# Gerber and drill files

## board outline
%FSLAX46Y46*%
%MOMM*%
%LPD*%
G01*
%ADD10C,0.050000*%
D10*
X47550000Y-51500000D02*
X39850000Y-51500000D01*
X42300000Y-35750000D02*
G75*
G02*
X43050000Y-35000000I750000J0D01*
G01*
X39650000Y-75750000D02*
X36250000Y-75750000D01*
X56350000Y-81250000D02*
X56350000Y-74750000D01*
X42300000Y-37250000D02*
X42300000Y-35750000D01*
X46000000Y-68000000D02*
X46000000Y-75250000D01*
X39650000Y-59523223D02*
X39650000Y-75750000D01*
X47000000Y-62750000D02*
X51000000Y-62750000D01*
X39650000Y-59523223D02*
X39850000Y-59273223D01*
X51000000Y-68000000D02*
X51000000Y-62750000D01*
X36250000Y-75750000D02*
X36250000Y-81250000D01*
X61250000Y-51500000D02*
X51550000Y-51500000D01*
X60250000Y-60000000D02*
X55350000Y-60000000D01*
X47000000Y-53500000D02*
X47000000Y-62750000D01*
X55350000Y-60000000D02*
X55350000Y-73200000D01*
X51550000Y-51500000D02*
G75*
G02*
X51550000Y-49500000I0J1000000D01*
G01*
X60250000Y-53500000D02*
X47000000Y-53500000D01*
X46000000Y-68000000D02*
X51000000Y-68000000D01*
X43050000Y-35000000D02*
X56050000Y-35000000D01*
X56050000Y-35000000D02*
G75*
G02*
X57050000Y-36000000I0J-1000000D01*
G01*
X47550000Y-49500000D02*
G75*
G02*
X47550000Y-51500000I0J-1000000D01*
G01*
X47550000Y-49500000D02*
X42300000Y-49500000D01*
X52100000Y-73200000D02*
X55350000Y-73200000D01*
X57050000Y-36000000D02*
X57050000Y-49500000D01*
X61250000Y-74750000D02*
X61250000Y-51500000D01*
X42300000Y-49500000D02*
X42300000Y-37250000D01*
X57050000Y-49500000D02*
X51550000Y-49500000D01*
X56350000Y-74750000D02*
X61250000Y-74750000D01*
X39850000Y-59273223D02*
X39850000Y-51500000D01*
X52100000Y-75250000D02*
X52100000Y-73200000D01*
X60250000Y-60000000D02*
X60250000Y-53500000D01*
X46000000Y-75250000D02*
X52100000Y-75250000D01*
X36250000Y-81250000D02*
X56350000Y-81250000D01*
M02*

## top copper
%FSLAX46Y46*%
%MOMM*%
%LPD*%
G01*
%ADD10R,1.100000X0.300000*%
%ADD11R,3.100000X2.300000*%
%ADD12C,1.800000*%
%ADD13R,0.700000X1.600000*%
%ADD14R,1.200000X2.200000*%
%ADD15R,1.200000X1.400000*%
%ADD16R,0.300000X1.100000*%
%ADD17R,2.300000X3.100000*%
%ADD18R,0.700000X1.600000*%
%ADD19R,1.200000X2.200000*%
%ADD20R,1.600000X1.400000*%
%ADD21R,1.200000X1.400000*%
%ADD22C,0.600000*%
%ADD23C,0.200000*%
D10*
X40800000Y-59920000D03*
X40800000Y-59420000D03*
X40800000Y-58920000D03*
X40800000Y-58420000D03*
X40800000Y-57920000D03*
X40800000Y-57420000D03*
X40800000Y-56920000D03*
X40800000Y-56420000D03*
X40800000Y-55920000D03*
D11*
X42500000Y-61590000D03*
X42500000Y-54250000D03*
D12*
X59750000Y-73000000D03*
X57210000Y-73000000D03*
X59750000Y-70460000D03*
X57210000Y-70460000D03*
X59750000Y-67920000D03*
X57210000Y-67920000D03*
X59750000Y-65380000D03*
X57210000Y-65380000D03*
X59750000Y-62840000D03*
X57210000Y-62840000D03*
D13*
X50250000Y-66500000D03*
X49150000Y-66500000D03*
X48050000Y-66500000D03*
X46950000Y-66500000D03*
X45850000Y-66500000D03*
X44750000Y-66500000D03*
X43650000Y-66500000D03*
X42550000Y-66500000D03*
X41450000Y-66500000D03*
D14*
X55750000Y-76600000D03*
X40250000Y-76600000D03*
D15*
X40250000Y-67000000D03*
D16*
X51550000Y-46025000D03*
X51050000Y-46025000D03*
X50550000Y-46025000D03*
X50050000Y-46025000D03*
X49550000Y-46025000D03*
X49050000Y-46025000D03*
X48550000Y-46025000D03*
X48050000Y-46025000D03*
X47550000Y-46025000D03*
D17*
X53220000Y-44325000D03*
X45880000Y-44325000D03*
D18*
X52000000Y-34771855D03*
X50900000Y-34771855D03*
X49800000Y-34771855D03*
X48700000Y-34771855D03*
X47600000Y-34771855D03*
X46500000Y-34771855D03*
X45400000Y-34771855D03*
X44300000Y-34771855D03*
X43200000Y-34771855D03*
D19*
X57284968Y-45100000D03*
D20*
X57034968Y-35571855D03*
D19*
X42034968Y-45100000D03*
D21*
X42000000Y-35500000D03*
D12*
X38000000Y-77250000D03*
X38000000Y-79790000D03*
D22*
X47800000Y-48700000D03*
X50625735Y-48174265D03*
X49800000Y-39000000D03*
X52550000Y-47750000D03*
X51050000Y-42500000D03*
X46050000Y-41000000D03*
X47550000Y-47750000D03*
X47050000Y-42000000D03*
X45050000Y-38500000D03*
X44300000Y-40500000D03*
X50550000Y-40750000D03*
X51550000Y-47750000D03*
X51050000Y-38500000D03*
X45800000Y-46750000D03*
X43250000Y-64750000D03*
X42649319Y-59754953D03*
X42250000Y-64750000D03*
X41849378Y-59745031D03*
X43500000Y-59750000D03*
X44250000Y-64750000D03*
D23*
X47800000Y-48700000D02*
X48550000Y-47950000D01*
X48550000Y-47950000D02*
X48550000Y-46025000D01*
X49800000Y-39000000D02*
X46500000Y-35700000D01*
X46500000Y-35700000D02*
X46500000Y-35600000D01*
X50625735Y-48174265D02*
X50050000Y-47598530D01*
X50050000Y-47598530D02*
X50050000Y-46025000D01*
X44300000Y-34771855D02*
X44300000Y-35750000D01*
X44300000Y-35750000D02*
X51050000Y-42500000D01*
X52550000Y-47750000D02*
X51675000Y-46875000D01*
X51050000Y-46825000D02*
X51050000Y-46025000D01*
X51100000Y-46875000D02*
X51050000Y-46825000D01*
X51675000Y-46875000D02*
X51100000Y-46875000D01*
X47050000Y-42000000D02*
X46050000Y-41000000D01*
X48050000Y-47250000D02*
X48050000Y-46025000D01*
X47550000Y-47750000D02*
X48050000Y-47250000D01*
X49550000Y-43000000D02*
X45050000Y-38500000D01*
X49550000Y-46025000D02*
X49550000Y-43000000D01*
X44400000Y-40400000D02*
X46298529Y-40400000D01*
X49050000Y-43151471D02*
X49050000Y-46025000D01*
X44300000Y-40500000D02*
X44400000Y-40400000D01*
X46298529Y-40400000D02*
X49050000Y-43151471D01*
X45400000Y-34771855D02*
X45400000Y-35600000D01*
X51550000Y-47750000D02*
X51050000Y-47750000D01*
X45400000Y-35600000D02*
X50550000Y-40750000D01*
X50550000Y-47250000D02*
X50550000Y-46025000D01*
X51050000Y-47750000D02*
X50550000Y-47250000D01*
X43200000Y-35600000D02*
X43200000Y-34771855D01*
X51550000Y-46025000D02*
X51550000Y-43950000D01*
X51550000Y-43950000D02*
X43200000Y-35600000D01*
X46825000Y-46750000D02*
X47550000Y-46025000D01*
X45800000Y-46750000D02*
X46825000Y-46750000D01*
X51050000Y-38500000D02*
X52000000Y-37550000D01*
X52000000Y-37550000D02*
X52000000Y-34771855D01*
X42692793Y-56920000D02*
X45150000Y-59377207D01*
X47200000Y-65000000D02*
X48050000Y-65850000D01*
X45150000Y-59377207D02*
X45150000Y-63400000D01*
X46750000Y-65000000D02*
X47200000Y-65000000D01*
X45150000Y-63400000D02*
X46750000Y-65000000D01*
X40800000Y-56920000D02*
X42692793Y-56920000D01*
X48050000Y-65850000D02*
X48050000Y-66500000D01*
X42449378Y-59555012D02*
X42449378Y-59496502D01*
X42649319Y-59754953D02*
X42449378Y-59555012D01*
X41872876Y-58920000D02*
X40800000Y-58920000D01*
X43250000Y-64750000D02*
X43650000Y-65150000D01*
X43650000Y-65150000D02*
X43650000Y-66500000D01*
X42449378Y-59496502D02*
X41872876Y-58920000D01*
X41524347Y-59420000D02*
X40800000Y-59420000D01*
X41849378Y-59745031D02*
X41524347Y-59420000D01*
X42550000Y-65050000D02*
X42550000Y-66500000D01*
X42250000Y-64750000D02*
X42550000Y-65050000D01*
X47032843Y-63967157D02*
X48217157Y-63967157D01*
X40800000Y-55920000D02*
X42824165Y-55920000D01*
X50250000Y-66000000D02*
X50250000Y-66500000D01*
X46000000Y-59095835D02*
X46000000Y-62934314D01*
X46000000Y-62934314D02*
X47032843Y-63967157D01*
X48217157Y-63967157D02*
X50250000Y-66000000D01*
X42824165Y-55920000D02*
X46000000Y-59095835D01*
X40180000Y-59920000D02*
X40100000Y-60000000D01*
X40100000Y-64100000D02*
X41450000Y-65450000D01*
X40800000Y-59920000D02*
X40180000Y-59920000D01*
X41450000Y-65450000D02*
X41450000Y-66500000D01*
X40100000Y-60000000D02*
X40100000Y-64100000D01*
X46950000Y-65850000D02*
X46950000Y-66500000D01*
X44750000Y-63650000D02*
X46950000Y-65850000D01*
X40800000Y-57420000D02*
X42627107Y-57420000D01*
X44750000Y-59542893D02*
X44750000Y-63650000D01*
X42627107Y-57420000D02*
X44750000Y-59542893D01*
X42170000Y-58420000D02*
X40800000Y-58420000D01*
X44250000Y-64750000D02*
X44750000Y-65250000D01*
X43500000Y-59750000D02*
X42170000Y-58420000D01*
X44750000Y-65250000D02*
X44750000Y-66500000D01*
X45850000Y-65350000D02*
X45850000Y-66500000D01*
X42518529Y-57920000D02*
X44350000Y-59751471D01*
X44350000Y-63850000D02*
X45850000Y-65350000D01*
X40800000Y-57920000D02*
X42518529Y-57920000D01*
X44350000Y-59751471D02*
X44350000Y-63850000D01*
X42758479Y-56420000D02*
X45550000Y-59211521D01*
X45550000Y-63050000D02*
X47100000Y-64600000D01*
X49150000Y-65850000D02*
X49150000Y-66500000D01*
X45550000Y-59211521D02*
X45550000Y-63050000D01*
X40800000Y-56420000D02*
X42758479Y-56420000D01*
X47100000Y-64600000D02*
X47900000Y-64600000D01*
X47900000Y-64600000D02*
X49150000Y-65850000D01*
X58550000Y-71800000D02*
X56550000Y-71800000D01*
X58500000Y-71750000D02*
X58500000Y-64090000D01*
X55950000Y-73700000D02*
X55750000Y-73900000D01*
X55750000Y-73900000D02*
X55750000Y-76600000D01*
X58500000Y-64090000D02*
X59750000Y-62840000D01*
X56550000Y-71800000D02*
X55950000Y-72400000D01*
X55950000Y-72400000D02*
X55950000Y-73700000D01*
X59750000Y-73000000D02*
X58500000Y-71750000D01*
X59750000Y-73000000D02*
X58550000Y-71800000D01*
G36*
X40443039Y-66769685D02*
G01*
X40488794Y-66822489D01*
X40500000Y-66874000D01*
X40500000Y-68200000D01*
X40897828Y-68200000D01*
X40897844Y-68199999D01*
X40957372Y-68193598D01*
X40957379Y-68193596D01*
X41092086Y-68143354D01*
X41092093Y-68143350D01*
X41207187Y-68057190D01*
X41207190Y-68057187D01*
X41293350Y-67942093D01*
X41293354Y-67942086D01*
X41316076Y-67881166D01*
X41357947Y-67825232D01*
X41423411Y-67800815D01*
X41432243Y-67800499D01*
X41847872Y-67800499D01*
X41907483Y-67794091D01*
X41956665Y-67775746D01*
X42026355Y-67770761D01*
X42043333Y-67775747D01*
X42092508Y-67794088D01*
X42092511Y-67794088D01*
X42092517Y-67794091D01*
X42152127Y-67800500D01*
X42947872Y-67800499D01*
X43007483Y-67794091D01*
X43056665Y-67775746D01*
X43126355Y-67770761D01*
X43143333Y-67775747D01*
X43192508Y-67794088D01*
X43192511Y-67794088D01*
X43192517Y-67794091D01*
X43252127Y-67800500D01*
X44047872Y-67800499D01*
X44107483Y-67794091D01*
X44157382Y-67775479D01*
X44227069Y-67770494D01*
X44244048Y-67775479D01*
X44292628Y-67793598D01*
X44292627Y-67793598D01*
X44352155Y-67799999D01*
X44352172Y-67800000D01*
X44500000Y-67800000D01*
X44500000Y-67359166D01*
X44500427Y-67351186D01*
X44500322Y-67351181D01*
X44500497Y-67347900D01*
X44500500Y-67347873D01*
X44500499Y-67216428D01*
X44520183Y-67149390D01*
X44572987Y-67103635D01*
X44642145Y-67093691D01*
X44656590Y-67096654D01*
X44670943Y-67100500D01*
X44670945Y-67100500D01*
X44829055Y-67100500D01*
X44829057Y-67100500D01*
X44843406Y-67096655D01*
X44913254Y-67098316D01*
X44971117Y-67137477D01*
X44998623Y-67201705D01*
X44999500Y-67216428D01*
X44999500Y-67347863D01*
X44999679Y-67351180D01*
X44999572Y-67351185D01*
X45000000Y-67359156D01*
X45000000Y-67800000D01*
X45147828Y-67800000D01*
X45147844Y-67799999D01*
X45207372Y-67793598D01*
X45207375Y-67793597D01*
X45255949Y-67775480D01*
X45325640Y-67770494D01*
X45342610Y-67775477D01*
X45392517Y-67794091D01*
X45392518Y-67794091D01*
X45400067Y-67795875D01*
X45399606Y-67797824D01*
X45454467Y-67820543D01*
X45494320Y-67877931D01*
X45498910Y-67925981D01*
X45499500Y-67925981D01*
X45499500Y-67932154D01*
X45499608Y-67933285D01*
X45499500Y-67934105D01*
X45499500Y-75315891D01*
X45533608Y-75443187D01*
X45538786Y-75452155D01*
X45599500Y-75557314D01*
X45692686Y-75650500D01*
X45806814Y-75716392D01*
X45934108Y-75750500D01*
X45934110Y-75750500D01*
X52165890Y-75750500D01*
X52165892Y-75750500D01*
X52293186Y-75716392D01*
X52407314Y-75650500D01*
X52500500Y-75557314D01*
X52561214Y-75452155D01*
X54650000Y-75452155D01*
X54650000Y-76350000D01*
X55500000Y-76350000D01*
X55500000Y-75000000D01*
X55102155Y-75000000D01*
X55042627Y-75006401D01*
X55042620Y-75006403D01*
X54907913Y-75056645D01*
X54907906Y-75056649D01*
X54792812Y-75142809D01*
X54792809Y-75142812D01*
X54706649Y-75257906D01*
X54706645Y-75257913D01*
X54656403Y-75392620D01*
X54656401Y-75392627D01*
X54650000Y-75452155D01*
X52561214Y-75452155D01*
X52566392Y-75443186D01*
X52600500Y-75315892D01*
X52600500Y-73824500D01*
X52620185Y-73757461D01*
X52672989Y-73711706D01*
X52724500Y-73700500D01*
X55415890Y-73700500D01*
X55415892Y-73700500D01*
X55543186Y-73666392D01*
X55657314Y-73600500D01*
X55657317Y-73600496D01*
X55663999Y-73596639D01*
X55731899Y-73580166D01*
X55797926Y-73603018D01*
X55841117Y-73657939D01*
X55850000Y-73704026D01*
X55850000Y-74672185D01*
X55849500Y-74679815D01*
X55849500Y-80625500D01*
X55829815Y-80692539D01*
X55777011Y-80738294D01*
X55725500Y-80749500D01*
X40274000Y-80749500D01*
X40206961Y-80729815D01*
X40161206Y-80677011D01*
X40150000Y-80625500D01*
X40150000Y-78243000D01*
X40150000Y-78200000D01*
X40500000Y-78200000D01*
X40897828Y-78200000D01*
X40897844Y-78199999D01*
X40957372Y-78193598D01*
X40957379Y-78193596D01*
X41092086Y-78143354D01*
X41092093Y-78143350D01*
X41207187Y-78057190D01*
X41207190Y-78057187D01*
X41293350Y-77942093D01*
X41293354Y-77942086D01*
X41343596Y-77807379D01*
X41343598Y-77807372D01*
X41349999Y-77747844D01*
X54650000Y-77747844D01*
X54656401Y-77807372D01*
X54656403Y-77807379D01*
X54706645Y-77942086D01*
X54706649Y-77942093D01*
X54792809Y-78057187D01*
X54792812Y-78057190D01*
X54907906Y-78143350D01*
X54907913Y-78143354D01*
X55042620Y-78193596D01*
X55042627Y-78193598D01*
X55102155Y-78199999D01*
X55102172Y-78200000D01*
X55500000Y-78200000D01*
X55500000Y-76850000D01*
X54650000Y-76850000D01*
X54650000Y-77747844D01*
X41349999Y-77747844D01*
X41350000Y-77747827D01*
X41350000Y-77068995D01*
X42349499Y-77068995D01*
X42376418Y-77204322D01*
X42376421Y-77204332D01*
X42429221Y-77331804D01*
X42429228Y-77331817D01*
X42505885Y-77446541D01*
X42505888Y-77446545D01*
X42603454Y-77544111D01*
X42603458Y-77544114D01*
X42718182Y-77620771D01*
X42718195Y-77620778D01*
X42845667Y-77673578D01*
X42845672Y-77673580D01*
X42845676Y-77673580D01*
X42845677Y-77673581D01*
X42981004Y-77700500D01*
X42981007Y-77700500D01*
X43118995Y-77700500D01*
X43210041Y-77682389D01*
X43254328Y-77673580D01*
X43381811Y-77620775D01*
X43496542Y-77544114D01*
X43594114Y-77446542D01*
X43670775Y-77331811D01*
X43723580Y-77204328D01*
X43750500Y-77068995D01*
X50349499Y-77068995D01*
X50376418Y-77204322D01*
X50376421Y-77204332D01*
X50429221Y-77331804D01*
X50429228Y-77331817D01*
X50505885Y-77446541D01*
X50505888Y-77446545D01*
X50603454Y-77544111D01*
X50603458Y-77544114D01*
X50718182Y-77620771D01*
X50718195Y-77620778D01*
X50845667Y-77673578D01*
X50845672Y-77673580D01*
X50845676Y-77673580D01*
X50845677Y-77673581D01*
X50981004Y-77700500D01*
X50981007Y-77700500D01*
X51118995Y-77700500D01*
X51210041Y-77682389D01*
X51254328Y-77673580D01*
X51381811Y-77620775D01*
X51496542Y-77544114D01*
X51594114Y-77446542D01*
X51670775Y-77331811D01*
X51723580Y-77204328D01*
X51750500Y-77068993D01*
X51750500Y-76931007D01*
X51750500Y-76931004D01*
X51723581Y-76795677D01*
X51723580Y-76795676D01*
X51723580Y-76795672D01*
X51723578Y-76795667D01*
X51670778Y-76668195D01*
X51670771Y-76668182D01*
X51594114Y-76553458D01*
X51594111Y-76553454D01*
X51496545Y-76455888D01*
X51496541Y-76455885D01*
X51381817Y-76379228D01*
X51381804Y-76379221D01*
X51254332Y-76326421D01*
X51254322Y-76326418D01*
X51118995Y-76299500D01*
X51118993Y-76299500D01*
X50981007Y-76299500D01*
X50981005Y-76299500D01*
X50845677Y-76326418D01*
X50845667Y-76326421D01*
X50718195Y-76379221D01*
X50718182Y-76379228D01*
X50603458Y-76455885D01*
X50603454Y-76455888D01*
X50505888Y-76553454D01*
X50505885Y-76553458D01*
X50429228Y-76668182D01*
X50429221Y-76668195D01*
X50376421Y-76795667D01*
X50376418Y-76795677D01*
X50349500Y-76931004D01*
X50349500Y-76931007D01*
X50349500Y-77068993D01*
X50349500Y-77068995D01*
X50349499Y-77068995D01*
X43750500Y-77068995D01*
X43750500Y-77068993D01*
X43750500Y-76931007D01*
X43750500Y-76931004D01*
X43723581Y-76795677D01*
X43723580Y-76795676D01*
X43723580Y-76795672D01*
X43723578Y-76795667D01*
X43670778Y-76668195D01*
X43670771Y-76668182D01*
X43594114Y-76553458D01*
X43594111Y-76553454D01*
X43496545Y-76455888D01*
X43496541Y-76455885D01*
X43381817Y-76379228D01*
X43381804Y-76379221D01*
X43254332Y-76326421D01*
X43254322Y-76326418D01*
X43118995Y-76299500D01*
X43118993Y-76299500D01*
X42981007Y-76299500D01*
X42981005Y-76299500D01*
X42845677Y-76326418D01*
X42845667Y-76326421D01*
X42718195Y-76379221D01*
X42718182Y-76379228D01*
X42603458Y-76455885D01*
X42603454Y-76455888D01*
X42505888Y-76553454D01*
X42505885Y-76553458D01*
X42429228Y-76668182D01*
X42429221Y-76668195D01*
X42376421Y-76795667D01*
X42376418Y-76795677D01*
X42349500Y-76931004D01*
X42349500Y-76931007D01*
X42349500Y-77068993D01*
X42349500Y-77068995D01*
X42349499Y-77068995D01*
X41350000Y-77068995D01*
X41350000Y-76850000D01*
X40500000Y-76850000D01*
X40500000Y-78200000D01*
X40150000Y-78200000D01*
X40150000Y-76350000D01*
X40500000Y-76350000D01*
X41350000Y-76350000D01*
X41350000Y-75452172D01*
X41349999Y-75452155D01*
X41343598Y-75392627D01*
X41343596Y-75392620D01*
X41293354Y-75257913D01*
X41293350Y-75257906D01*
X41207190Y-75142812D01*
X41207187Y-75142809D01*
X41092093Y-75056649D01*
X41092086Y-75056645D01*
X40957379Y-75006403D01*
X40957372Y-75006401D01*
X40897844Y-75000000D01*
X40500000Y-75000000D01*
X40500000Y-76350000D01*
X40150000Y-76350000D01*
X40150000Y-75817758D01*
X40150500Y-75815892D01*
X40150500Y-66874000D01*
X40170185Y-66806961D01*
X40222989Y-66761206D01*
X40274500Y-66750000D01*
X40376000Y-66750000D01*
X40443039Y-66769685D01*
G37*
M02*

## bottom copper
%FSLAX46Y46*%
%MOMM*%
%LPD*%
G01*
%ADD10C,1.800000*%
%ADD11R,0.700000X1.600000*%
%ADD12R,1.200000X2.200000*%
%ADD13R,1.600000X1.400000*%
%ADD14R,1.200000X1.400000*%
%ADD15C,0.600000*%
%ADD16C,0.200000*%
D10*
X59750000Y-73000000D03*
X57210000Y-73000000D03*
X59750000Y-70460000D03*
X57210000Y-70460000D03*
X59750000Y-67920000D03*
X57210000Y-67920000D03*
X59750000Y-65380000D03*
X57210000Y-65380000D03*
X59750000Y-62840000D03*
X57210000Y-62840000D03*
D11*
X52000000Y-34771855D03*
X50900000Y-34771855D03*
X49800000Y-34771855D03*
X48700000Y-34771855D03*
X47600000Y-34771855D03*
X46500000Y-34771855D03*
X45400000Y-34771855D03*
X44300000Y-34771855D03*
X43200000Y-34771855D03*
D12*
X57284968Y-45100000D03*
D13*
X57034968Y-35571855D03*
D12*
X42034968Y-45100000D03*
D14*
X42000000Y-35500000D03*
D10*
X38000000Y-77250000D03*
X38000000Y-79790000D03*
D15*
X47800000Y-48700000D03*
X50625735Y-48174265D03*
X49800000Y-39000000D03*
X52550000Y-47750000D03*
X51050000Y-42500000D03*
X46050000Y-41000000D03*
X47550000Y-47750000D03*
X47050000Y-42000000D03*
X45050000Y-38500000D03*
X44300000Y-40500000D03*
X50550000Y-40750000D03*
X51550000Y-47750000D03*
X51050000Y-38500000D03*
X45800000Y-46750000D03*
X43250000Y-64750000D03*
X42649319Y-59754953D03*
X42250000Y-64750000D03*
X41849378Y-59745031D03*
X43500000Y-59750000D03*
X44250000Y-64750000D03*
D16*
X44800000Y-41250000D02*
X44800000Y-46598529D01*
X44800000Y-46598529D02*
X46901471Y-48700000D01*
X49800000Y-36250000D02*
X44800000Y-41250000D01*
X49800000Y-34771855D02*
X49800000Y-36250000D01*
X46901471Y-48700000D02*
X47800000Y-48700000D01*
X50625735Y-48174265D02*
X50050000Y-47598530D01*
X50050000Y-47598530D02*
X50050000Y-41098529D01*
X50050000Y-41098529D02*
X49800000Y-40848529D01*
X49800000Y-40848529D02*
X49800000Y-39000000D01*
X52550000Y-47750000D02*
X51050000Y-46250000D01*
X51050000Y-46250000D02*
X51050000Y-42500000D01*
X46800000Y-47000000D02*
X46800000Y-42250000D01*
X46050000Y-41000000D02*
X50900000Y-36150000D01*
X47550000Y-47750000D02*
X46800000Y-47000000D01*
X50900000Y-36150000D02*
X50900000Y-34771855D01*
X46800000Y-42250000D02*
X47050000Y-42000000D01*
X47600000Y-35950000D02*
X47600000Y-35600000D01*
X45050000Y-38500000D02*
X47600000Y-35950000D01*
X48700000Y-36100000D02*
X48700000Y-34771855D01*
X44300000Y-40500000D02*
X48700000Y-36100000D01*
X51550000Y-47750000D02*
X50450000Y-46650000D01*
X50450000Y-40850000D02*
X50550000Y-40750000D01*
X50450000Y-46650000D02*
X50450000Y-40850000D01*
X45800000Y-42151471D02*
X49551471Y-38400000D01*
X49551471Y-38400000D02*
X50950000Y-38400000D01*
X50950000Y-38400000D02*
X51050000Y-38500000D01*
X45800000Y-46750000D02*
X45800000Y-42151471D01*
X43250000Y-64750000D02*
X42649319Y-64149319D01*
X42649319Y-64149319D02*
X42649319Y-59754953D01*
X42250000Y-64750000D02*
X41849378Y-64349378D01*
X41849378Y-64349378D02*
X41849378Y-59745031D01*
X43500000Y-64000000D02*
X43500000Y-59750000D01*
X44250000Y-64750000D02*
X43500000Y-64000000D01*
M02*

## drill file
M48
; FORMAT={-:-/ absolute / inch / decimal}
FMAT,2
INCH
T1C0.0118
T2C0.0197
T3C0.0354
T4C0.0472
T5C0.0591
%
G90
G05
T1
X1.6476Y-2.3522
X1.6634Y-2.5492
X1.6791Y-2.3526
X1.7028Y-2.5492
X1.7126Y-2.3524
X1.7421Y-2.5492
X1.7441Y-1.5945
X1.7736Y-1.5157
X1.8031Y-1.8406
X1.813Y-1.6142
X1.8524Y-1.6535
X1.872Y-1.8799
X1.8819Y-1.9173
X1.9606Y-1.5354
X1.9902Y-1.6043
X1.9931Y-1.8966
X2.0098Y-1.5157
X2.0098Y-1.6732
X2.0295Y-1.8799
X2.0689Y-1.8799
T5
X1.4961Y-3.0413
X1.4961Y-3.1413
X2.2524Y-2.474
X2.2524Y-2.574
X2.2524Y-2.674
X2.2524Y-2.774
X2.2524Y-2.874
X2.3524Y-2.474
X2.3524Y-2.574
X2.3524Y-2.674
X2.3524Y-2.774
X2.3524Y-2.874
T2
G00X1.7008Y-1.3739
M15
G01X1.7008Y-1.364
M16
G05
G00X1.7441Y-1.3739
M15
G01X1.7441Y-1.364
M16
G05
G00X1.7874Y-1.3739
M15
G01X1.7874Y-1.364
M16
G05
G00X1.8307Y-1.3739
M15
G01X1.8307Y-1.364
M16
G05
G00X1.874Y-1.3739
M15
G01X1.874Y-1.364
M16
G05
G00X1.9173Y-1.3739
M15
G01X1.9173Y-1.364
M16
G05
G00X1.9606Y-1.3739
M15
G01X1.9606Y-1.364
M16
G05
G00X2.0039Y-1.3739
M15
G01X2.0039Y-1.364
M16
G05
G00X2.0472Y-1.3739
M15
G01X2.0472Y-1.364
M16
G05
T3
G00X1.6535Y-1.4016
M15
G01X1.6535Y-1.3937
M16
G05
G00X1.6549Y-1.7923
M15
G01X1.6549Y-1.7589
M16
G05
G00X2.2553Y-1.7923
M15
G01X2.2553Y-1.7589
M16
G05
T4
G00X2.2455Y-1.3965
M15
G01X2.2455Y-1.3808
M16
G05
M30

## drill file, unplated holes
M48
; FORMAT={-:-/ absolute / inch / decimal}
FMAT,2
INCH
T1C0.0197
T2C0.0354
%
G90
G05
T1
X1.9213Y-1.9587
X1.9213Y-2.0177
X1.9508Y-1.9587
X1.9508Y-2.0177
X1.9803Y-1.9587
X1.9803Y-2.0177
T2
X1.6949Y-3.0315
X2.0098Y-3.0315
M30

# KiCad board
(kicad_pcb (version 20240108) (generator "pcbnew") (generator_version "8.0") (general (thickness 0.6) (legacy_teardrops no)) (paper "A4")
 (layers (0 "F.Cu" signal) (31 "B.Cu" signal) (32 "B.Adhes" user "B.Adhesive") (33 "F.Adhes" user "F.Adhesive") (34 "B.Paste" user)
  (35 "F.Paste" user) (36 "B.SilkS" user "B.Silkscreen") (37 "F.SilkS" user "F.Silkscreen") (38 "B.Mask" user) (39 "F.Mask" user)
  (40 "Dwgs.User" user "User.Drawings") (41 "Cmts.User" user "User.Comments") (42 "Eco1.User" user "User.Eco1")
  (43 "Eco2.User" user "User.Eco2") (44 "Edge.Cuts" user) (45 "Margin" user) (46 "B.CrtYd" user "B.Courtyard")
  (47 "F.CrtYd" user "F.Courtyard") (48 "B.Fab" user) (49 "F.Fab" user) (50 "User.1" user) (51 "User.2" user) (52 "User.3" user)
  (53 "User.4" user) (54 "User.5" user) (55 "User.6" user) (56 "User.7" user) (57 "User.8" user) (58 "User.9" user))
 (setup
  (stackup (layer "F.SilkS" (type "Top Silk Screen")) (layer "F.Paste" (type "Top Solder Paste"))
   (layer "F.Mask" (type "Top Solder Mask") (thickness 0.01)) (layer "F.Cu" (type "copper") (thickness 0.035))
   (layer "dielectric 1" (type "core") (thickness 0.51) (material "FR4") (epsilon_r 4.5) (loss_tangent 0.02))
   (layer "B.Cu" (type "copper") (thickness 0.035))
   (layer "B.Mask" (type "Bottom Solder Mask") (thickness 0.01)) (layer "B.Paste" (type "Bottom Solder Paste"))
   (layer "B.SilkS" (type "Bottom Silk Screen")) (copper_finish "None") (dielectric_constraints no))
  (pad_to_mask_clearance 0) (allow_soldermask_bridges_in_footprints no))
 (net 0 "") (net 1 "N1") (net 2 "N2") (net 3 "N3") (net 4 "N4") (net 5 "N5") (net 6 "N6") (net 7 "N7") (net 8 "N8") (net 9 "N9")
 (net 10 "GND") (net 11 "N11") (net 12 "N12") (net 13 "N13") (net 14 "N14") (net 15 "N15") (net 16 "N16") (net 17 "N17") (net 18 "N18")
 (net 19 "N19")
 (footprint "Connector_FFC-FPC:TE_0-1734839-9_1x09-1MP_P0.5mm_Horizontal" (layer "F.Cu") (at 42.15 57.92 90)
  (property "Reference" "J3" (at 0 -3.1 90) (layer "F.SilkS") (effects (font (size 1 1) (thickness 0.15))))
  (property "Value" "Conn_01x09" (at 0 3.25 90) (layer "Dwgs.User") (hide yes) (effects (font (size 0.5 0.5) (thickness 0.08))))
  (pad "1" smd rect (at -2 -1.35 90) (size 0.3 1.1) (layers "F.Cu" "F.Paste" "F.Mask") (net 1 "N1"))
  (pad "2" smd rect (at -1.5 -1.35 90) (size 0.3 1.1) (layers "F.Cu" "F.Paste" "F.Mask") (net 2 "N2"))
  (pad "3" smd rect (at -1 -1.35 90) (size 0.3 1.1) (layers "F.Cu" "F.Paste" "F.Mask") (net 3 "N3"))
  (pad "4" smd rect (at -0.5 -1.35 90) (size 0.3 1.1) (layers "F.Cu" "F.Paste" "F.Mask") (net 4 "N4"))
  (pad "5" smd rect (at 0 -1.35 90) (size 0.3 1.1) (layers "F.Cu" "F.Paste" "F.Mask") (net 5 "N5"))
  (pad "6" smd rect (at 0.5 -1.35 90) (size 0.3 1.1) (layers "F.Cu" "F.Paste" "F.Mask") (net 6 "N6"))
  (pad "7" smd rect (at 1 -1.35 90) (size 0.3 1.1) (layers "F.Cu" "F.Paste" "F.Mask") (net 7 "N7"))
  (pad "8" smd rect (at 1.5 -1.35 90) (size 0.3 1.1) (layers "F.Cu" "F.Paste" "F.Mask") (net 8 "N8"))
  (pad "9" smd rect (at 2 -1.35 90) (size 0.3 1.1) (layers "F.Cu" "F.Paste" "F.Mask") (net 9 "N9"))
  (pad "MP" smd rect (at -3.67 0.35 90) (size 2.3 3.1) (layers "F.Cu" "F.Paste" "F.Mask"))
  (pad "MP" smd rect (at 3.67 0.35 90) (size 2.3 3.1) (layers "F.Cu" "F.Paste" "F.Mask")))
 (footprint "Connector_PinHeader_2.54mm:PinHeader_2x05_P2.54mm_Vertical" (layer "F.Cu") (at 59.75 73 180)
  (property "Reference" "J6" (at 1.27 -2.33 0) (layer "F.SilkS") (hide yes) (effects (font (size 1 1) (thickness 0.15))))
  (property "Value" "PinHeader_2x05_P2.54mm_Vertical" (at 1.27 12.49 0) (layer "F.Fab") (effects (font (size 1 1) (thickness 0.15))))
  (pad "1" thru_hole circle (at 0 0 180) (size 1.8 1.8) (drill 1.5) (layers "*.Cu" "*.Mask") (remove_unused_layers no) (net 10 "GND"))
  (pad "2" thru_hole circle (at 2.54 0 180) (size 1.8 1.8) (drill 1.5) (layers "*.Cu" "*.Mask") (remove_unused_layers no)
   (thermal_bridge_angle 90))
  (pad "3" thru_hole circle (at 0 2.54 180) (size 1.8 1.8) (drill 1.5) (layers "*.Cu" "*.Mask") (remove_unused_layers no)
   (thermal_bridge_angle 90))
  (pad "4" thru_hole circle (at 2.54 2.54 180) (size 1.8 1.8) (drill 1.5) (layers "*.Cu" "*.Mask") (remove_unused_layers no)
   (thermal_bridge_angle 90))
  (pad "5" thru_hole circle (at 0 5.08 180) (size 1.8 1.8) (drill 1.5) (layers "*.Cu" "*.Mask") (remove_unused_layers no)
   (thermal_bridge_angle 90))
  (pad "6" thru_hole circle (at 2.54 5.08 180) (size 1.8 1.8) (drill 1.5) (layers "*.Cu" "*.Mask") (remove_unused_layers no)
   (thermal_bridge_angle 90))
  (pad "7" thru_hole circle (at 0 7.62 180) (size 1.8 1.8) (drill 1.5) (layers "*.Cu" "*.Mask") (remove_unused_layers no)
   (thermal_bridge_angle 90))
  (pad "8" thru_hole circle (at 2.54 7.62 180) (size 1.8 1.8) (drill 1.5) (layers "*.Cu" "*.Mask") (remove_unused_layers no)
   (thermal_bridge_angle 90))
  (pad "9" thru_hole circle (at 0 10.16 180) (size 1.8 1.8) (drill 1.5) (layers "*.Cu" "*.Mask") (remove_unused_layers no) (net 10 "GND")
   (thermal_bridge_angle 90))
  (pad "10" thru_hole circle (at 2.54 10.16 180) (size 1.8 1.8) (drill 1.5) (layers "*.Cu" "*.Mask") (remove_unused_layers no)
   (thermal_bridge_angle 90)))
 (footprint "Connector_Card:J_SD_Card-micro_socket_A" (layer "F.Cu") (at 47.034968 73.521855 180)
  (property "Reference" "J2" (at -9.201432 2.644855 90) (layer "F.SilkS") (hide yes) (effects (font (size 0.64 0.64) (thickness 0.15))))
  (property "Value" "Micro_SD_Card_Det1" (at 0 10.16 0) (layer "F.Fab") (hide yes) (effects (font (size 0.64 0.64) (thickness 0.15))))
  (pad "" np_thru_hole circle (at -4.015032 -3.478145 180) (size 0.9 0.9) (drill 0.9) (layers "*.Cu" "*.Mask"))
  (pad "" np_thru_hole circle (at 3.984968 -3.478145 180) (size 0.9 0.9) (drill 0.9) (layers "*.Cu" "*.Mask"))
  (pad "1" smd rect (at -3.215032 7.021855 180) (size 0.7 1.6) (layers "F.Cu" "F.Paste" "F.Mask") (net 9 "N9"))
  (pad "2" smd rect (at -2.115032 7.021855 180) (size 0.7 1.6) (layers "F.Cu" "F.Paste" "F.Mask") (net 8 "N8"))
  (pad "3" smd rect (at -1.015032 7.021855 180) (size 0.7 1.6) (layers "F.Cu" "F.Paste" "F.Mask") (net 7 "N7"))
  (pad "4" smd rect (at 0.084968 7.021855 180) (size 0.7 1.6) (layers "F.Cu" "F.Paste" "F.Mask") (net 6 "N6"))
  (pad "5" smd rect (at 1.184968 7.021855 180) (size 0.7 1.6) (layers "F.Cu" "F.Paste" "F.Mask") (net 5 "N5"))
  (pad "6" smd rect (at 2.284968 7.021855 180) (size 0.7 1.6) (layers "F.Cu" "F.Paste" "F.Mask") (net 10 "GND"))
  (pad "7" smd rect (at 3.384968 7.021855 180) (size 0.7 1.6) (layers "F.Cu" "F.Paste" "F.Mask") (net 3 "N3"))
  (pad "8" smd rect (at 4.484968 7.021855 180) (size 0.7 1.6) (layers "F.Cu" "F.Paste" "F.Mask") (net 2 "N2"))
  (pad "9" smd rect (at 5.584968 7.021855 180) (size 0.7 1.6) (layers "F.Cu" "F.Paste" "F.Mask") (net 1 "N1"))
  (pad "SH" smd rect (at -8.715032 -3.078145 180) (size 1.2 2.2) (layers "F.Cu" "F.Paste" "F.Mask") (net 10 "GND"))
  (pad "SH" smd rect (at 6.784968 -3.078145 180) (size 1.2 2.2) (layers "F.Cu" "F.Paste" "F.Mask") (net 10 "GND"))
  (pad "SH" smd rect (at 6.784968 6.521855 180) (size 1.2 1.4) (layers "F.Cu" "F.Paste" "F.Mask") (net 10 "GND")))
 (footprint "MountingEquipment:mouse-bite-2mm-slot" (layer "F.Cu") (at 49.55 50.5)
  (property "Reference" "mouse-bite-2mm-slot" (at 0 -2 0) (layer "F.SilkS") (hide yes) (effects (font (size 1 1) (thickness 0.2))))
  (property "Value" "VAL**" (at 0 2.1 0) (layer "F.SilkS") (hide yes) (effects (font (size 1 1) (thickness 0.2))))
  (pad "" np_thru_hole circle (at -0.75 -0.75) (size 0.5 0.5) (drill 0.5) (layers "*.Cu" "*.Mask"))
  (pad "" np_thru_hole circle (at -0.75 0.75) (size 0.5 0.5) (drill 0.5) (layers "*.Cu" "*.Mask"))
  (pad "" np_thru_hole circle (at 0 -0.75) (size 0.5 0.5) (drill 0.5) (layers "*.Cu" "*.Mask"))
  (pad "" np_thru_hole circle (at 0 0.75) (size 0.5 0.5) (drill 0.5) (layers "*.Cu" "*.Mask"))
  (pad "" np_thru_hole circle (at 0.75 -0.75) (size 0.5 0.5) (drill 0.5) (layers "*.Cu" "*.Mask"))
  (pad "" np_thru_hole circle (at 0.75 0.75) (size 0.5 0.5) (drill 0.5) (layers "*.Cu" "*.Mask")))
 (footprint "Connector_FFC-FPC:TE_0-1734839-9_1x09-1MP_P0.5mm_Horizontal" (layer "F.Cu") (at 49.55 44.675 180)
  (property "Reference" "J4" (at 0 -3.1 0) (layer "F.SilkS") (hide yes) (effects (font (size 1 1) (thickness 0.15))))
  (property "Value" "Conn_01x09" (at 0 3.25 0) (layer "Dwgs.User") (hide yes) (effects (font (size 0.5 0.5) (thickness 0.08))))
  (pad "1" smd rect (at -2 -1.35 180) (size 0.3 1.1) (layers "F.Cu" "F.Paste" "F.Mask") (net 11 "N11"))
  (pad "2" smd rect (at -1.5 -1.35 180) (size 0.3 1.1) (layers "F.Cu" "F.Paste" "F.Mask") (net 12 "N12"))
  (pad "3" smd rect (at -1 -1.35 180) (size 0.3 1.1) (layers "F.Cu" "F.Paste" "F.Mask") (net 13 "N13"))
  (pad "4" smd rect (at -0.5 -1.35 180) (size 0.3 1.1) (layers "F.Cu" "F.Paste" "F.Mask") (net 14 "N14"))
  (pad "5" smd rect (at 0 -1.35 180) (size 0.3 1.1) (layers "F.Cu" "F.Paste" "F.Mask") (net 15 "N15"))
  (pad "6" smd rect (at 0.5 -1.35 180) (size 0.3 1.1) (layers "F.Cu" "F.Paste" "F.Mask") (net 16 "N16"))
  (pad "7" smd rect (at 1 -1.35 180) (size 0.3 1.1) (layers "F.Cu" "F.Paste" "F.Mask") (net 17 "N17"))
  (pad "8" smd rect (at 1.5 -1.35 180) (size 0.3 1.1) (layers "F.Cu" "F.Paste" "F.Mask") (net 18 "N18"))
  (pad "9" smd rect (at 2 -1.35 180) (size 0.3 1.1) (layers "F.Cu" "F.Paste" "F.Mask") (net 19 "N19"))
  (pad "MP" smd rect (at -3.67 0.35 180) (size 2.3 3.1) (layers "F.Cu" "F.Paste" "F.Mask"))
  (pad "MP" smd rect (at 3.67 0.35 180) (size 2.3 3.1) (layers "F.Cu" "F.Paste" "F.Mask")))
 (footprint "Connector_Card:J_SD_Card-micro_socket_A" (layer "F.Cu") (at 48.784968 42.021855 180)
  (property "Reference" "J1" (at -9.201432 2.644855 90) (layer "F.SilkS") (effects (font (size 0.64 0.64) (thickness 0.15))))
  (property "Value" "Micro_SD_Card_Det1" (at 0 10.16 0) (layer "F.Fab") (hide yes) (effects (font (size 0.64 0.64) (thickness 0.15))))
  (pad "1" thru_hole rect (at -3.215032 7.25 180) (size 0.7 1.6) (drill oval 0.5 0.75) (layers "*.Cu" "*.Mask") (remove_unused_layers no)
   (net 19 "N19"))
  (pad "2" thru_hole rect (at -2.115032 7.25 180) (size 0.7 1.6) (drill oval 0.5 0.75) (layers "*.Cu" "*.Mask") (remove_unused_layers no)
   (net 18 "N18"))
  (pad "3" thru_hole rect (at -1.015032 7.25 180) (size 0.7 1.6) (drill oval 0.5 0.75) (layers "*.Cu" "*.Mask") (remove_unused_layers no)
   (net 17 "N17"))
  (pad "4" thru_hole rect (at 0.084968 7.25 180) (size 0.7 1.6) (drill oval 0.5 0.75) (layers "*.Cu" "*.Mask") (remove_unused_layers no)
   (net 16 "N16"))
  (pad "5" thru_hole rect (at 1.184968 7.25 180) (size 0.7 1.6) (drill oval 0.5 0.75) (layers "*.Cu" "*.Mask") (remove_unused_layers no)
   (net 15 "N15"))
  (pad "6" thru_hole rect (at 2.284968 7.25 180) (size 0.7 1.6) (drill oval 0.5 0.75) (layers "*.Cu" "*.Mask") (remove_unused_layers no)
   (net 14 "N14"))
  (pad "7" thru_hole rect (at 3.384968 7.25 180) (size 0.7 1.6) (drill oval 0.5 0.75) (layers "*.Cu" "*.Mask") (remove_unused_layers no)
   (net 13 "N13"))
  (pad "8" thru_hole rect (at 4.484968 7.25 180) (size 0.7 1.6) (drill oval 0.5 0.75) (layers "*.Cu" "*.Mask") (remove_unused_layers no)
   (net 12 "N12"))
  (pad "9" thru_hole rect (at 5.584968 7.25 180) (size 0.7 1.6) (drill oval 0.5 0.75) (layers "*.Cu" "*.Mask") (remove_unused_layers no)
   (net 11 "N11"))
  (pad "SH" thru_hole rect (at -8.5 -3.078145 180) (size 1.2 2.2) (drill oval 0.9 1.75) (layers "*.Cu" "*.Mask") (remove_unused_layers no))
  (pad "SH" thru_hole rect (at -8.25 6.75 180) (size 1.6 1.4) (drill oval 1.2 1.6 (offset 0 -0.3)) (layers "*.Cu" "*.Mask")
   (remove_unused_layers no))
  (pad "SH" thru_hole rect (at 6.75 -3.078145 180) (size 1.2 2.2) (drill oval 0.9 1.75) (layers "*.Cu" "*.Mask") (remove_unused_layers no))
  (pad "SH" thru_hole rect (at 6.784968 6.521855 180) (size 1.2 1.4) (drill oval 0.9 1.1) (layers "*.Cu" "*.Mask") (remove_unused_layers no)))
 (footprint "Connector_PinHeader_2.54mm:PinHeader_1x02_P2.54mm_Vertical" (layer "F.Cu") (at 38 77.25)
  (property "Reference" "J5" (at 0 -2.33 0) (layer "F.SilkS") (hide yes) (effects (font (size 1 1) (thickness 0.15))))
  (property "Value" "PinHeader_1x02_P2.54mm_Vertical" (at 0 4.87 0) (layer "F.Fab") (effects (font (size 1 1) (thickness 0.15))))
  (pad "1" thru_hole circle (at 0 0) (size 1.8 1.8) (drill 1.5) (layers "*.Cu" "*.Mask") (remove_unused_layers no) (thermal_bridge_angle 90))
  (pad "2" thru_hole circle (at 0 2.54) (size 1.8 1.8) (drill 1.5) (layers "*.Cu" "*.Mask") (remove_unused_layers no)
   (thermal_bridge_angle 90)))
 (gr_line (start 47.55 51.5) (end 39.85 51.5) (stroke (width 0.05) (type default)) (layer "Edge.Cuts"))
 (gr_arc (start 42.3 35.75) (mid 42.51967 35.21967) (end 43.05 35) (stroke (width 0.05) (type default)) (layer "Edge.Cuts"))
 (gr_line (start 39.65 75.75) (end 36.25 75.75) (stroke (width 0.05) (type default)) (layer "Edge.Cuts"))
 (gr_line (start 56.35 81.25) (end 56.35 74.75) (stroke (width 0.05) (type default)) (layer "Edge.Cuts"))
 (gr_line (start 42.3 37.25) (end 42.3 35.75) (stroke (width 0.05) (type default)) (layer "Edge.Cuts"))
 (gr_line (start 46 68) (end 46 75.25) (stroke (width 0.05) (type default)) (layer "Edge.Cuts"))
 (gr_line (start 39.65 59.523223) (end 39.65 75.75) (stroke (width 0.05) (type default)) (layer "Edge.Cuts"))
 (gr_line (start 47 62.75) (end 51 62.75) (stroke (width 0.05) (type default)) (layer "Edge.Cuts"))
 (gr_line (start 39.65 59.523223) (end 39.85 59.273223) (stroke (width 0.05) (type default)) (layer "Edge.Cuts"))
 (gr_line (start 51 68) (end 51 62.75) (stroke (width 0.05) (type default)) (layer "Edge.Cuts"))
 (gr_line (start 36.25 75.75) (end 36.25 81.25) (stroke (width 0.05) (type default)) (layer "Edge.Cuts"))
 (gr_line (start 61.25 51.5) (end 51.55 51.5) (stroke (width 0.05) (type default)) (layer "Edge.Cuts"))
 (gr_line (start 60.25 60) (end 55.35 60) (stroke (width 0.05) (type default)) (layer "Edge.Cuts"))
 (gr_line (start 47 53.5) (end 47 62.75) (stroke (width 0.05) (type default)) (layer "Edge.Cuts"))
 (gr_line (start 55.35 60) (end 55.35 73.2) (stroke (width 0.05) (type default)) (layer "Edge.Cuts"))
 (gr_arc (start 51.55 51.5) (mid 50.55 50.5) (end 51.55 49.5) (stroke (width 0.05) (type default)) (layer "Edge.Cuts"))
 (gr_line (start 60.25 53.5) (end 47 53.5) (stroke (width 0.05) (type default)) (layer "Edge.Cuts"))
 (gr_line (start 46 68) (end 51 68) (stroke (width 0.05) (type default)) (layer "Edge.Cuts"))
 (gr_line (start 43.05 35) (end 56.05 35) (stroke (width 0.05) (type default)) (layer "Edge.Cuts"))
 (gr_arc (start 56.05 35) (mid 56.757107 35.292893) (end 57.05 36) (stroke (width 0.05) (type default)) (layer "Edge.Cuts"))
 (gr_arc (start 47.55 49.5) (mid 48.55 50.5) (end 47.55 51.5) (stroke (width 0.05) (type default)) (layer "Edge.Cuts"))
 (gr_line (start 47.55 49.5) (end 42.3 49.5) (stroke (width 0.05) (type default)) (layer "Edge.Cuts"))
 (gr_line (start 52.1 73.2) (end 55.35 73.2) (stroke (width 0.05) (type default)) (layer "Edge.Cuts"))
 (gr_line (start 57.05 36) (end 57.05 49.5) (stroke (width 0.05) (type default)) (layer "Edge.Cuts"))
 (gr_line (start 61.25 74.75) (end 61.25 51.5) (stroke (width 0.05) (type default)) (layer "Edge.Cuts"))
 (gr_line (start 42.3 49.5) (end 42.3 37.25) (stroke (width 0.05) (type default)) (layer "Edge.Cuts"))
 (gr_line (start 57.05 49.5) (end 51.55 49.5) (stroke (width 0.05) (type default)) (layer "Edge.Cuts"))
 (gr_line (start 56.35 74.75) (end 61.25 74.75) (stroke (width 0.05) (type default)) (layer "Edge.Cuts"))
 (gr_line (start 39.85 59.273223) (end 39.85 51.5) (stroke (width 0.05) (type default)) (layer "Edge.Cuts"))
 (gr_line (start 52.1 75.25) (end 52.1 73.2) (stroke (width 0.05) (type default)) (layer "Edge.Cuts"))
 (gr_line (start 60.25 60) (end 60.25 53.5) (stroke (width 0.05) (type default)) (layer "Edge.Cuts"))
 (gr_line (start 46 75.25) (end 52.1 75.25) (stroke (width 0.05) (type default)) (layer "Edge.Cuts"))
 (gr_line (start 36.25 81.25) (end 56.35 81.25) (stroke (width 0.05) (type default)) (layer "Edge.Cuts"))
 (segment (start 47.8 48.7) (end 48.55 47.95) (width 0.2) (layer "F.Cu") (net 17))
 (segment (start 48.55 47.95) (end 48.55 46.025) (width 0.2) (layer "F.Cu") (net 17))
 (via (at 47.8 48.7) (size 0.6) (drill 0.3) (layers "F.Cu" "B.Cu") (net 17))
 (segment (start 44.8 41.25) (end 44.8 46.598529) (width 0.2) (layer "B.Cu") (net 17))
 (segment (start 44.8 46.598529) (end 46.901471 48.7) (width 0.2) (layer "B.Cu") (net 17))
 (segment (start 49.8 36.25) (end 44.8 41.25) (width 0.2) (layer "B.Cu") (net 17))
 (segment (start 49.8 34.771855) (end 49.8 36.25) (width 0.2) (layer "B.Cu") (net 17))
 (segment (start 46.901471 48.7) (end 47.8 48.7) (width 0.2) (layer "B.Cu") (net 17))
 (segment (start 49.8 39) (end 46.5 35.7) (width 0.2) (layer "F.Cu") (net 14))
 (segment (start 46.5 35.7) (end 46.5 35.6) (width 0.2) (layer "F.Cu") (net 14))
 (segment (start 50.625735 48.174265) (end 50.05 47.59853) (width 0.2) (layer "F.Cu") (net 14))
 (segment (start 50.05 47.59853) (end 50.05 46.025) (width 0.2) (layer "F.Cu") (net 14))
 (via (at 50.625735 48.174265) (size 0.6) (drill 0.3) (layers "F.Cu" "B.Cu") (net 14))
 (via (at 49.8 39) (size 0.6) (drill 0.3) (layers "F.Cu" "B.Cu") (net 14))
 (segment (start 50.625735 48.174265) (end 50.05 47.59853) (width 0.2) (layer "B.Cu") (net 14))
 (segment (start 50.05 47.59853) (end 50.05 41.098529) (width 0.2) (layer "B.Cu") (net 14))
 (segment (start 50.05 41.098529) (end 49.8 40.848529) (width 0.2) (layer "B.Cu") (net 14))
 (segment (start 49.8 40.848529) (end 49.8 39) (width 0.2) (layer "B.Cu") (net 14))
 (segment (start 44.3 34.771855) (end 44.3 35.75) (width 0.2) (layer "F.Cu") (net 12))
 (segment (start 44.3 35.75) (end 51.05 42.5) (width 0.2) (layer "F.Cu") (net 12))
 (segment (start 52.55 47.75) (end 51.675 46.875) (width 0.2) (layer "F.Cu") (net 12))
 (segment (start 51.05 46.825) (end 51.05 46.025) (width 0.2) (layer "F.Cu") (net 12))
 (segment (start 51.1 46.875) (end 51.05 46.825) (width 0.2) (layer "F.Cu") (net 12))
 (segment (start 51.675 46.875) (end 51.1 46.875) (width 0.2) (layer "F.Cu") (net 12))
 (via (at 52.55 47.75) (size 0.6) (drill 0.3) (layers "F.Cu" "B.Cu") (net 12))
 (via (at 51.05 42.5) (size 0.6) (drill 0.3) (layers "F.Cu" "B.Cu") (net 12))
 (segment (start 52.55 47.75) (end 51.05 46.25) (width 0.2) (layer "B.Cu") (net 12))
 (segment (start 51.05 46.25) (end 51.05 42.5) (width 0.2) (layer "B.Cu") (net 12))
 (segment (start 47.05 42) (end 46.05 41) (width 0.2) (layer "F.Cu") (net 18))
 (segment (start 48.05 47.25) (end 48.05 46.025) (width 0.2) (layer "F.Cu") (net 18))
 (segment (start 47.55 47.75) (end 48.05 47.25) (width 0.2) (layer "F.Cu") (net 18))
 (via (at 46.05 41) (size 0.6) (drill 0.3) (layers "F.Cu" "B.Cu") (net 18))
 (via (at 47.55 47.75) (size 0.6) (drill 0.3) (layers "F.Cu" "B.Cu") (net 18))
 (via (at 47.05 42) (size 0.6) (drill 0.3) (layers "F.Cu" "B.Cu") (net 18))
 (segment (start 46.8 47) (end 46.8 42.25) (width 0.2) (layer "B.Cu") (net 18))
 (segment (start 46.05 41) (end 50.9 36.15) (width 0.2) (layer "B.Cu") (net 18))
 (segment (start 47.55 47.75) (end 46.8 47) (width 0.2) (layer "B.Cu") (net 18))
 (segment (start 50.9 36.15) (end 50.9 34.771855) (width 0.2) (layer "B.Cu") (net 18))
 (segment (start 46.8 42.25) (end 47.05 42) (width 0.2) (layer "B.Cu") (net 18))
 (segment (start 49.55 43) (end 45.05 38.5) (width 0.2) (layer "F.Cu") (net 15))
 (segment (start 49.55 46.025) (end 49.55 43) (width 0.2) (layer "F.Cu") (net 15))
 (via (at 45.05 38.5) (size 0.6) (drill 0.3) (layers "F.Cu" "B.Cu") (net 15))
 (segment (start 47.6 35.95) (end 47.6 35.6) (width 0.2) (layer "B.Cu") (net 15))
 (segment (start 45.05 38.5) (end 47.6 35.95) (width 0.2) (layer "B.Cu") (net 15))
 (segment (start 44.4 40.4) (end 46.298529 40.4) (width 0.2) (layer "F.Cu") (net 16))
 (segment (start 49.05 43.151471) (end 49.05 46.025) (width 0.2) (layer "F.Cu") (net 16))
 (segment (start 44.3 40.5) (end 44.4 40.4) (width 0.2) (layer "F.Cu") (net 16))
 (segment (start 46.298529 40.4) (end 49.05 43.151471) (width 0.2) (layer "F.Cu") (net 16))
 (via (at 44.3 40.5) (size 0.6) (drill 0.3) (layers "F.Cu" "B.Cu") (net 16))
 (segment (start 48.7 36.1) (end 48.7 34.771855) (width 0.2) (layer "B.Cu") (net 16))
 (segment (start 44.3 40.5) (end 48.7 36.1) (width 0.2) (layer "B.Cu") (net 16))
 (segment (start 45.4 34.771855) (end 45.4 35.6) (width 0.2) (layer "F.Cu") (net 13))
 (segment (start 51.55 47.75) (end 51.05 47.75) (width 0.2) (layer "F.Cu") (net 13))
 (segment (start 45.4 35.6) (end 50.55 40.75) (width 0.2) (layer "F.Cu") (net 13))
 (segment (start 50.55 47.25) (end 50.55 46.025) (width 0.2) (layer "F.Cu") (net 13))
 (segment (start 51.05 47.75) (end 50.55 47.25) (width 0.2) (layer "F.Cu") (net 13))
 (via (at 50.55 40.75) (size 0.6) (drill 0.3) (layers "F.Cu" "B.Cu") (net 13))
 (via (at 51.55 47.75) (size 0.6) (drill 0.3) (layers "F.Cu" "B.Cu") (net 13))
 (segment (start 51.55 47.75) (end 50.45 46.65) (width 0.2) (layer "B.Cu") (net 13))
 (segment (start 50.45 40.85) (end 50.55 40.75) (width 0.2) (layer "B.Cu") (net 13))
 (segment (start 50.45 46.65) (end 50.45 40.85) (width 0.2) (layer "B.Cu") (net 13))
 (segment (start 43.2 35.6) (end 43.2 34.771855) (width 0.2) (layer "F.Cu") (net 11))
 (segment (start 51.55 46.025) (end 51.55 43.95) (width 0.2) (layer "F.Cu") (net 11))
 (segment (start 51.55 43.95) (end 43.2 35.6) (width 0.2) (layer "F.Cu") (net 11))
 (segment (start 46.825 46.75) (end 47.55 46.025) (width 0.2) (layer "F.Cu") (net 19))
 (segment (start 45.8 46.75) (end 46.825 46.75) (width 0.2) (layer "F.Cu") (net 19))
 (segment (start 51.05 38.5) (end 52 37.55) (width 0.2) (layer "F.Cu") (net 19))
 (segment (start 52 37.55) (end 52 34.771855) (width 0.2) (layer "F.Cu") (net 19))
 (via (at 51.05 38.5) (size 0.6) (drill 0.3) (layers "F.Cu" "B.Cu") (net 19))
 (via (at 45.8 46.75) (size 0.6) (drill 0.3) (layers "F.Cu" "B.Cu") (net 19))
 (segment (start 45.8 42.151471) (end 49.551471 38.4) (width 0.2) (layer "B.Cu") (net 19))
 (segment (start 49.551471 38.4) (end 50.95 38.4) (width 0.2) (layer "B.Cu") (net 19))
 (segment (start 50.95 38.4) (end 51.05 38.5) (width 0.2) (layer "B.Cu") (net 19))
 (segment (start 45.8 46.75) (end 45.8 42.151471) (width 0.2) (layer "B.Cu") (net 19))
 (segment (start 42.692793 56.92) (end 45.15 59.377207) (width 0.2) (layer "F.Cu") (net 7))
 (segment (start 47.2 65) (end 48.05 65.85) (width 0.2) (layer "F.Cu") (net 7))
 (segment (start 45.15 59.377207) (end 45.15 63.4) (width 0.2) (layer "F.Cu") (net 7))
 (segment (start 46.75 65) (end 47.2 65) (width 0.2) (layer "F.Cu") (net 7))
 (segment (start 45.15 63.4) (end 46.75 65) (width 0.2) (layer "F.Cu") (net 7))
 (segment (start 40.8 56.92) (end 42.692793 56.92) (width 0.2) (layer "F.Cu") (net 7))
 (segment (start 48.05 65.85) (end 48.05 66.5) (width 0.2) (layer "F.Cu") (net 7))
 (segment (start 42.449378 59.555012) (end 42.449378 59.496502) (width 0.2) (layer "F.Cu") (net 3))
 (segment (start 42.649319 59.754953) (end 42.449378 59.555012) (width 0.2) (layer "F.Cu") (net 3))
 (segment (start 41.872876 58.92) (end 40.8 58.92) (width 0.2) (layer "F.Cu") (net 3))
 (segment (start 43.25 64.75) (end 43.65 65.15) (width 0.2) (layer "F.Cu") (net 3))
 (segment (start 43.65 65.15) (end 43.65 66.5) (width 0.2) (layer "F.Cu") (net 3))
 (segment (start 42.449378 59.496502) (end 41.872876 58.92) (width 0.2) (layer "F.Cu") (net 3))
 (via (at 43.25 64.75) (size 0.6) (drill 0.3) (layers "F.Cu" "B.Cu") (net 3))
 (via (at 42.649319 59.754953) (size 0.6) (drill 0.3) (layers "F.Cu" "B.Cu") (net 3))
 (segment (start 43.25 64.75) (end 42.649319 64.149319) (width 0.2) (layer "B.Cu") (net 3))
 (segment (start 42.649319 64.149319) (end 42.649319 59.754953) (width 0.2) (layer "B.Cu") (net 3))
 (segment (start 41.524347 59.42) (end 40.8 59.42) (width 0.2) (layer "F.Cu") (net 2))
 (segment (start 41.849378 59.745031) (end 41.524347 59.42) (width 0.2) (layer "F.Cu") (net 2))
 (segment (start 42.55 65.05) (end 42.55 66.5) (width 0.2) (layer "F.Cu") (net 2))
 (segment (start 42.25 64.75) (end 42.55 65.05) (width 0.2) (layer "F.Cu") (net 2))
 (via (at 42.25 64.75) (size 0.6) (drill 0.3) (layers "F.Cu" "B.Cu") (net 2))
 (via (at 41.849378 59.745031) (size 0.6) (drill 0.3) (layers "F.Cu" "B.Cu") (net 2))
 (segment (start 42.25 64.75) (end 41.849378 64.349378) (width 0.2) (layer "B.Cu") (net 2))
 (segment (start 41.849378 64.349378) (end 41.849378 59.745031) (width 0.2) (layer "B.Cu") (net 2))
 (segment (start 47.032843 63.967157) (end 48.217157 63.967157) (width 0.2) (layer "F.Cu") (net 9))
 (segment (start 40.8 55.92) (end 42.824165 55.92) (width 0.2) (layer "F.Cu") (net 9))
 (segment (start 50.25 66) (end 50.25 66.5) (width 0.2) (layer "F.Cu") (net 9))
 (segment (start 46 59.095835) (end 46 62.934314) (width 0.2) (layer "F.Cu") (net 9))
 (segment (start 46 62.934314) (end 47.032843 63.967157) (width 0.2) (layer "F.Cu") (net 9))
 (segment (start 48.217157 63.967157) (end 50.25 66) (width 0.2) (layer "F.Cu") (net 9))
 (segment (start 42.824165 55.92) (end 46 59.095835) (width 0.2) (layer "F.Cu") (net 9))
 (segment (start 40.18 59.92) (end 40.1 60) (width 0.2) (layer "F.Cu") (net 1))
 (segment (start 40.1 64.1) (end 41.45 65.45) (width 0.2) (layer "F.Cu") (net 1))
 (segment (start 40.8 59.92) (end 40.18 59.92) (width 0.2) (layer "F.Cu") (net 1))
 (segment (start 41.45 65.45) (end 41.45 66.5) (width 0.2) (layer "F.Cu") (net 1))
 (segment (start 40.1 60) (end 40.1 64.1) (width 0.2) (layer "F.Cu") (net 1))
 (segment (start 46.95 65.85) (end 46.95 66.5) (width 0.2) (layer "F.Cu") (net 6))
 (segment (start 44.75 63.65) (end 46.95 65.85) (width 0.2) (layer "F.Cu") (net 6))
 (segment (start 40.8 57.42) (end 42.627107 57.42) (width 0.2) (layer "F.Cu") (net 6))
 (segment (start 44.75 59.542893) (end 44.75 63.65) (width 0.2) (layer "F.Cu") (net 6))
 (segment (start 42.627107 57.42) (end 44.75 59.542893) (width 0.2) (layer "F.Cu") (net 6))
 (segment (start 42.17 58.42) (end 40.8 58.42) (width 0.2) (layer "F.Cu") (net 4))
 (segment (start 44.25 64.75) (end 44.75 65.25) (width 0.2) (layer "F.Cu") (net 4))
 (segment (start 43.5 59.75) (end 42.17 58.42) (width 0.2) (layer "F.Cu") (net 4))
 (segment (start 44.75 65.25) (end 44.75 66.5) (width 0.2) (layer "F.Cu") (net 4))
 (via (at 43.5 59.75) (size 0.6) (drill 0.3) (layers "F.Cu" "B.Cu") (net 4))
 (via (at 44.25 64.75) (size 0.6) (drill 0.3) (layers "F.Cu" "B.Cu") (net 4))
 (segment (start 43.5 64) (end 43.5 59.75) (width 0.2) (layer "B.Cu") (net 4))
 (segment (start 44.25 64.75) (end 43.5 64) (width 0.2) (layer "B.Cu") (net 4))
 (segment (start 45.85 65.35) (end 45.85 66.5) (width 0.2) (layer "F.Cu") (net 5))
 (segment (start 42.518529 57.92) (end 44.35 59.751471) (width 0.2) (layer "F.Cu") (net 5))
 (segment (start 44.35 63.85) (end 45.85 65.35) (width 0.2) (layer "F.Cu") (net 5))
 (segment (start 40.8 57.92) (end 42.518529 57.92) (width 0.2) (layer "F.Cu") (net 5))
 (segment (start 44.35 59.751471) (end 44.35 63.85) (width 0.2) (layer "F.Cu") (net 5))
 (segment (start 42.758479 56.42) (end 45.55 59.211521) (width 0.2) (layer "F.Cu") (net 8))
 (segment (start 45.55 63.05) (end 47.1 64.6) (width 0.2) (layer "F.Cu") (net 8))
 (segment (start 49.15 65.85) (end 49.15 66.5) (width 0.2) (layer "F.Cu") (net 8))
 (segment (start 45.55 59.211521) (end 45.55 63.05) (width 0.2) (layer "F.Cu") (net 8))
 (segment (start 40.8 56.42) (end 42.758479 56.42) (width 0.2) (layer "F.Cu") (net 8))
 (segment (start 47.1 64.6) (end 47.9 64.6) (width 0.2) (layer "F.Cu") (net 8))
 (segment (start 47.9 64.6) (end 49.15 65.85) (width 0.2) (layer "F.Cu") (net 8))
 (segment (start 58.55 71.8) (end 56.55 71.8) (width 0.2) (layer "F.Cu") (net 10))
 (segment (start 58.5 71.75) (end 58.5 64.09) (width 0.2) (layer "F.Cu") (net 10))
 (segment (start 55.95 73.7) (end 55.75 73.9) (width 0.2) (layer "F.Cu") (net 10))
 (segment (start 55.75 73.9) (end 55.75 76.6) (width 0.2) (layer "F.Cu") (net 10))
 (segment (start 58.5 64.09) (end 59.75 62.84) (width 0.2) (layer "F.Cu") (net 10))
 (segment (start 56.55 71.8) (end 55.95 72.4) (width 0.2) (layer "F.Cu") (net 10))
 (segment (start 55.95 72.4) (end 55.95 73.7) (width 0.2) (layer "F.Cu") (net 10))
 (segment (start 59.75 73) (end 58.5 71.75) (width 0.2) (layer "F.Cu") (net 10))
 (segment (start 59.75 73) (end 58.55 71.8) (width 0.2) (layer "F.Cu") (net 10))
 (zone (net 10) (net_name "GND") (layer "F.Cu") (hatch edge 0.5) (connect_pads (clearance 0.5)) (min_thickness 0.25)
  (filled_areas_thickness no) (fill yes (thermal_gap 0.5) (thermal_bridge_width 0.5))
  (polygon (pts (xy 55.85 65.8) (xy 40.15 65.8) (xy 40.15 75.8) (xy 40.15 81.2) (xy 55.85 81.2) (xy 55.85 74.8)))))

